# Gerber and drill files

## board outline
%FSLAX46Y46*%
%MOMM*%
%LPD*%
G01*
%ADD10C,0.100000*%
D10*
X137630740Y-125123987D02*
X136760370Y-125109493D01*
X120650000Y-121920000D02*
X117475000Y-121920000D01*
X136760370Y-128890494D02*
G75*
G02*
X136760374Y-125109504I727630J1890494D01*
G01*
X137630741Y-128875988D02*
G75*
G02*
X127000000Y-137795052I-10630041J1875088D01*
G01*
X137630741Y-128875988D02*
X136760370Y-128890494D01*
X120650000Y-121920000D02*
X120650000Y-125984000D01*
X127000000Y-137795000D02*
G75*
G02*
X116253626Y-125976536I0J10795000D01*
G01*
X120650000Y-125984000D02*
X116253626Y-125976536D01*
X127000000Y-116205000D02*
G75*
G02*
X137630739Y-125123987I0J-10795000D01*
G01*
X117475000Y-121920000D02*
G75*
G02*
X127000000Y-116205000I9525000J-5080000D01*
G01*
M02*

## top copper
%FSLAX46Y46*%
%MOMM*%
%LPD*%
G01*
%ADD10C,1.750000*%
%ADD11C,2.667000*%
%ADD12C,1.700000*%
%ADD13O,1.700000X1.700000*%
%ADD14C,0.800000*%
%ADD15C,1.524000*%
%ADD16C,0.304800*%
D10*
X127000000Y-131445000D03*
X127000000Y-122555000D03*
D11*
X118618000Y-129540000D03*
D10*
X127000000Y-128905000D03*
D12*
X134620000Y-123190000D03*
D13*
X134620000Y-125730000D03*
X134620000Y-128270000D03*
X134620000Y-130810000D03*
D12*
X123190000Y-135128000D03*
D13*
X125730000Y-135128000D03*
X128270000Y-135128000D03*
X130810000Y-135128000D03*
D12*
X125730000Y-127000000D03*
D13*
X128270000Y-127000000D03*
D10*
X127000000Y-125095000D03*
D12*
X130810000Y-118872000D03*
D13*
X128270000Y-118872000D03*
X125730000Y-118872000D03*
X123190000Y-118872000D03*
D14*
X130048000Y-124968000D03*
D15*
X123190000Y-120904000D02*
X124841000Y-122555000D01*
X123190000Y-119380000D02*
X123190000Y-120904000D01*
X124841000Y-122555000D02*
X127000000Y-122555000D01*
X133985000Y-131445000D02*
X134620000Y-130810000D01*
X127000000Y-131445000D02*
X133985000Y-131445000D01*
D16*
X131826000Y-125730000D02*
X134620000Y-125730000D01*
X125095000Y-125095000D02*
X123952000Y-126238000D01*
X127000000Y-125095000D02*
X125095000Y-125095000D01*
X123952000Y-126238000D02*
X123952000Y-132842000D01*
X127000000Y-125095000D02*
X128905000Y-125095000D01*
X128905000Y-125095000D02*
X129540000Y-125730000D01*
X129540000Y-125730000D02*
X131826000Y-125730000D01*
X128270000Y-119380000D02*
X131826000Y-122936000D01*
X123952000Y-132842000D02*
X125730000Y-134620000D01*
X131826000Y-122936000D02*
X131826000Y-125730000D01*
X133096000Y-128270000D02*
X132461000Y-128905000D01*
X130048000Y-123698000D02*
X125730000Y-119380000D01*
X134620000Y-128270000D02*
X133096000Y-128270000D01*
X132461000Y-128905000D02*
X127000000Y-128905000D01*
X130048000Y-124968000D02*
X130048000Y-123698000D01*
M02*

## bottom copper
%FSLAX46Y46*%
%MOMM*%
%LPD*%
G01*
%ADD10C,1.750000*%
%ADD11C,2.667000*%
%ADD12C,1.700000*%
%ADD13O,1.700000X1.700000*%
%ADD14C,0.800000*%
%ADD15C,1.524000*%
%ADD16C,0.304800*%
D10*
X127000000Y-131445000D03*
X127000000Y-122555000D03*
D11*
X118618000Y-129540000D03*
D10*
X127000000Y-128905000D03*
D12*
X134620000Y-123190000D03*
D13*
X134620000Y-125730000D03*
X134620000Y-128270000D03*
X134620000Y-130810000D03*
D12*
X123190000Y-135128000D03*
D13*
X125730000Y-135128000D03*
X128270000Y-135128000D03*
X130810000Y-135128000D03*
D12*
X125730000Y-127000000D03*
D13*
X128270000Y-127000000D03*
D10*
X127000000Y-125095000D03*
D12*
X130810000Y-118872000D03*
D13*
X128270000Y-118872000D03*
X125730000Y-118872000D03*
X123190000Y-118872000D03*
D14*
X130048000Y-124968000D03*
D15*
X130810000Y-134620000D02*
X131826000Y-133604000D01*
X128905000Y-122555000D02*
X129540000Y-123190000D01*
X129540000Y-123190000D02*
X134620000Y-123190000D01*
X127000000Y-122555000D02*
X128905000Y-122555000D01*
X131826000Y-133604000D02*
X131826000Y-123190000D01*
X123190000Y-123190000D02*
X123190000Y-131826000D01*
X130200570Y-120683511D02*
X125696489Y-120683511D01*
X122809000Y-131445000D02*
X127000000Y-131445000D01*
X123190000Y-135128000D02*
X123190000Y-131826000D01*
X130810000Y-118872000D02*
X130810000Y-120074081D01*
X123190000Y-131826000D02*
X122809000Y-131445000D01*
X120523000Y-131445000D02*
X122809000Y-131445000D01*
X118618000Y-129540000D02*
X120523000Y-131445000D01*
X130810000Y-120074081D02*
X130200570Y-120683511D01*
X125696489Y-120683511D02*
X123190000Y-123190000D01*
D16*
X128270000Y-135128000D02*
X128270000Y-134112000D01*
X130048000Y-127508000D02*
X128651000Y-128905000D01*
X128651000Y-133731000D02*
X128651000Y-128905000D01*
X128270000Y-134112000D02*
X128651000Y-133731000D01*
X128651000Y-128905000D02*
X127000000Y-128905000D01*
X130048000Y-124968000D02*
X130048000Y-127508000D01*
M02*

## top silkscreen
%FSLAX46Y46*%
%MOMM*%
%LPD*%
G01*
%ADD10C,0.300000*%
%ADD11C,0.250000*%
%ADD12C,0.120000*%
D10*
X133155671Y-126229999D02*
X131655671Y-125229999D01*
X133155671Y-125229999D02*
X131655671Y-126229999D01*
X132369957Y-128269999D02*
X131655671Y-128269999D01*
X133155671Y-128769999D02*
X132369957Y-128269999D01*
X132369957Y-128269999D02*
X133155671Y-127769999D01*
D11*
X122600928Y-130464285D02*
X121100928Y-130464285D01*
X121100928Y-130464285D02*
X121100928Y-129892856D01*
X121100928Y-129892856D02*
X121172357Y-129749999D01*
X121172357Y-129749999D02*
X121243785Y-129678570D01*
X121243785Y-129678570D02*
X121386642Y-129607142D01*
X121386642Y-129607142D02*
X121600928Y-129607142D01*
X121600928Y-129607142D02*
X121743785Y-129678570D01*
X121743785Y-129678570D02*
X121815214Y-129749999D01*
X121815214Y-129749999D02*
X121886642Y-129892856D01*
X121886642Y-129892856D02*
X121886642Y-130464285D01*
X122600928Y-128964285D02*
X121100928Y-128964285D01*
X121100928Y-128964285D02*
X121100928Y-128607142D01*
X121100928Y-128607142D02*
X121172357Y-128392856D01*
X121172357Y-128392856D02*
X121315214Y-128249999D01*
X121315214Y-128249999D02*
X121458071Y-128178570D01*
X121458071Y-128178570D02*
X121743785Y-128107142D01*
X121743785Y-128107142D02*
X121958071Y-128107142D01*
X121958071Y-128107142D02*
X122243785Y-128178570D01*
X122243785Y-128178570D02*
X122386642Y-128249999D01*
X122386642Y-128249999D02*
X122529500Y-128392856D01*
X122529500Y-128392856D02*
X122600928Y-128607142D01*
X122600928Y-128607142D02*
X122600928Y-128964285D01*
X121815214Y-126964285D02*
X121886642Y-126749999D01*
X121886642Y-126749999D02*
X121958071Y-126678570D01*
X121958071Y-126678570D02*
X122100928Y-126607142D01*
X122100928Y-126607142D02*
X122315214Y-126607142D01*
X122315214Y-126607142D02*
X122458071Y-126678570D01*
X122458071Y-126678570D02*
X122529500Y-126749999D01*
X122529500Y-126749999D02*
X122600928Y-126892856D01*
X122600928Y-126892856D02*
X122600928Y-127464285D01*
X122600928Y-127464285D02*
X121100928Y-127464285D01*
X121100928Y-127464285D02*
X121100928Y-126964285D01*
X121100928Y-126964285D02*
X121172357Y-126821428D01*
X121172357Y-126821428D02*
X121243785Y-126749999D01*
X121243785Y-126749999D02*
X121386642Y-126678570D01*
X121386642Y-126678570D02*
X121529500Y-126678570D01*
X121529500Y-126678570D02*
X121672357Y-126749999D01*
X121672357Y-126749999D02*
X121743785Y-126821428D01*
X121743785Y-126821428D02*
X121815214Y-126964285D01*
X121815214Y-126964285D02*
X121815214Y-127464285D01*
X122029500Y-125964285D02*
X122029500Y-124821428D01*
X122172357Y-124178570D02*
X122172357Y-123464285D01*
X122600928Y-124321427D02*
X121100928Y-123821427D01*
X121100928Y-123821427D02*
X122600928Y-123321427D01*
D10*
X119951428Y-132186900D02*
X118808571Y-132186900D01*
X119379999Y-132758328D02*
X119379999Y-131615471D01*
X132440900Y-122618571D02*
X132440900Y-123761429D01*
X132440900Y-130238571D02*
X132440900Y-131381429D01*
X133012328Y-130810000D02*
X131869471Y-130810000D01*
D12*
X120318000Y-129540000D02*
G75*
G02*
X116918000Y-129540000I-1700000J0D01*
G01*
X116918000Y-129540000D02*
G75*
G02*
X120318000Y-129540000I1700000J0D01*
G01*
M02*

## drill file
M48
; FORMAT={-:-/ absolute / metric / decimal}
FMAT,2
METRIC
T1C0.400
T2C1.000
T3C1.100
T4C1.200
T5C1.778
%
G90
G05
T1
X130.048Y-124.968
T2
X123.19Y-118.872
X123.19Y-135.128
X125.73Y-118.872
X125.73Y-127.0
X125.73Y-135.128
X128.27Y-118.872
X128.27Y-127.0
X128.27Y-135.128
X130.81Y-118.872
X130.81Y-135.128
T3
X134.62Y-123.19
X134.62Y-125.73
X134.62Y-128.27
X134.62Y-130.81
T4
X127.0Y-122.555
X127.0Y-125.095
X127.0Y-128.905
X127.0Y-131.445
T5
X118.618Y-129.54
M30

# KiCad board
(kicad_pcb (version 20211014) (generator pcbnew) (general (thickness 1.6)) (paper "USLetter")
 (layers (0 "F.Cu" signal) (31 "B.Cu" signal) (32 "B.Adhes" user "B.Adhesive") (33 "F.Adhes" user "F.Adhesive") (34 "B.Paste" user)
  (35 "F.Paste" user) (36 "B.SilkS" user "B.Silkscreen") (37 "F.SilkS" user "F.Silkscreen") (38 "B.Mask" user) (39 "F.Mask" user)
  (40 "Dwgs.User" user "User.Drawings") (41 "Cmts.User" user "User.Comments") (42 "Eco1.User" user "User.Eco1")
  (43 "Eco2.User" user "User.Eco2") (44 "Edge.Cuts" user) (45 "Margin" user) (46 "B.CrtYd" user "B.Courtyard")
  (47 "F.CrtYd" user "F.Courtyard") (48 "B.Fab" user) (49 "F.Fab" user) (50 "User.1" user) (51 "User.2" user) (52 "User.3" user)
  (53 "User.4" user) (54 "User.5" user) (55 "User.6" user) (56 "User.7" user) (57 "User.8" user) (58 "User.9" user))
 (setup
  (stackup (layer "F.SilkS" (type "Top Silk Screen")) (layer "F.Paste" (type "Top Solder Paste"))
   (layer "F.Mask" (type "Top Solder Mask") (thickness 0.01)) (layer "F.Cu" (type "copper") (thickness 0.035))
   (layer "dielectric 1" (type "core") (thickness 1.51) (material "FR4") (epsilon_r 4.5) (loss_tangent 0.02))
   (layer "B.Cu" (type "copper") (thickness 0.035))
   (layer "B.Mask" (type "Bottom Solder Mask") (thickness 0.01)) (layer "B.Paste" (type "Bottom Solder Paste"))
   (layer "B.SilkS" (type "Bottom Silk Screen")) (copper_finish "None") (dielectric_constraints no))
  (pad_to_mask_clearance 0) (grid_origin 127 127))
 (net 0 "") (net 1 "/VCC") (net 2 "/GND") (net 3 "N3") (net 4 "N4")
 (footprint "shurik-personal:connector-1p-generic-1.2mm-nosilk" (layer "F.Cu") (at 127 131.445)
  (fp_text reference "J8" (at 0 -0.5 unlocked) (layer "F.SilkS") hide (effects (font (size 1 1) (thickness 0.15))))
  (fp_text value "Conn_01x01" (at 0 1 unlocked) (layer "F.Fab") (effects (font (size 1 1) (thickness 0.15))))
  (pad "1" thru_hole circle (at 0 0) (size 1.75 1.75) (drill 1.2) (layers *.Cu *.Mask) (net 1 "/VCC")))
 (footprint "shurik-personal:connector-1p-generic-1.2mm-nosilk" (layer "F.Cu") (at 127 122.555)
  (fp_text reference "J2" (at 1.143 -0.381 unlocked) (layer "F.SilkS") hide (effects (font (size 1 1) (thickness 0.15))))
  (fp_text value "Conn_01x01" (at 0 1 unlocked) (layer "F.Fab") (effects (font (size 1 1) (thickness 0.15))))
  (pad "1" thru_hole circle (at 0 0) (size 1.75 1.75) (drill 1.2) (layers *.Cu *.Mask) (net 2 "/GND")))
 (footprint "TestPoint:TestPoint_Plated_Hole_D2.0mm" (layer "F.Cu") (at 118.618 129.54)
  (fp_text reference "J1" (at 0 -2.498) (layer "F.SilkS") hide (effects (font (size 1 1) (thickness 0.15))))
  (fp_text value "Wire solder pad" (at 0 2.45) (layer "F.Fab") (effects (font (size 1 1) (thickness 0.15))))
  (fp_circle (center 0 0) (end 0 -1.7) (layer "F.SilkS") (width 0.12) (fill none))
  (pad "1" thru_hole circle (at 0 0) (size 2.667 2.667) (drill 1.778) (layers *.Cu *.Mask) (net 1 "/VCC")))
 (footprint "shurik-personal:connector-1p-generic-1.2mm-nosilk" (layer "F.Cu") (at 127 128.905)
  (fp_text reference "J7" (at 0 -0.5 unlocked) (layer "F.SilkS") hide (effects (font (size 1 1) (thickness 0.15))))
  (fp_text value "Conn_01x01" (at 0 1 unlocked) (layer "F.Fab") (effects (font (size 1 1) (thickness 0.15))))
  (pad "1" thru_hole circle (at 0 0) (size 1.75 1.75) (drill 1.2) (layers *.Cu *.Mask) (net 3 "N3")))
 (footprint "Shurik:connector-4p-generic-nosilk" (layer "F.Cu") (at 134.62 123.19)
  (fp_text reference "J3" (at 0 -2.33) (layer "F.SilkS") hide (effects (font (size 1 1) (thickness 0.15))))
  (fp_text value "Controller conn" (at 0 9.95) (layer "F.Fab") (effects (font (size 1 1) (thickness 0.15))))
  (pad "1" thru_hole circle (at 0 0) (size 1.7 1.7) (drill 1.1) (layers *.Cu *.Mask) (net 2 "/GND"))
  (pad "2" thru_hole oval (at 0 2.54) (size 1.7 1.7) (drill 1.1) (layers *.Cu *.Mask) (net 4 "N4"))
  (pad "3" thru_hole oval (at 0 5.08) (size 1.7 1.7) (drill 1.1) (layers *.Cu *.Mask) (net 3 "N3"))
  (pad "4" thru_hole oval (at 0 7.62) (size 1.7 1.7) (drill 1.1) (layers *.Cu *.Mask) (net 1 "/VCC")))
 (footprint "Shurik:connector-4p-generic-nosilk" (layer "F.Cu") (at 123.19 135.128 90)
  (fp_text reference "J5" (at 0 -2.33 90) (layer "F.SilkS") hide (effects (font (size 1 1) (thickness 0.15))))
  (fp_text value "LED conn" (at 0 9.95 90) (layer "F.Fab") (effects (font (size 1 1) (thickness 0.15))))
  (pad "1" thru_hole circle (at 0 0 90) (size 1.7 1.7) (drill 1) (layers *.Cu *.Mask) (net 1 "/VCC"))
  (pad "2" thru_hole oval (at 0 2.54 90) (size 1.7 1.7) (drill 1) (layers *.Cu *.Mask) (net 4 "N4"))
  (pad "3" thru_hole oval (at 0 5.08 90) (size 1.7 1.7) (drill 1) (layers *.Cu *.Mask) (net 3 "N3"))
  (pad "4" thru_hole oval (at 0 7.62 90) (size 1.7 1.7) (drill 1) (layers *.Cu *.Mask) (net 2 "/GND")))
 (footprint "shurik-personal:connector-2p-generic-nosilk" (layer "F.Cu") (at 125.73 127 90)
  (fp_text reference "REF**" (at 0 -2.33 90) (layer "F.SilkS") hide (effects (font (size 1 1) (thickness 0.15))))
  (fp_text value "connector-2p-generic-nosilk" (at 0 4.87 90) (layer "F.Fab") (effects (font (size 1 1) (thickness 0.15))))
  (pad "1" thru_hole circle (at 0 0 90) (size 1.7 1.7) (drill 1) (layers *.Cu *.Mask))
  (pad "2" thru_hole oval (at 0 2.54 90) (size 1.7 1.7) (drill 1) (layers *.Cu *.Mask)))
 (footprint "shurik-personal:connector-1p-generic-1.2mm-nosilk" (layer "F.Cu") (at 127 125.095)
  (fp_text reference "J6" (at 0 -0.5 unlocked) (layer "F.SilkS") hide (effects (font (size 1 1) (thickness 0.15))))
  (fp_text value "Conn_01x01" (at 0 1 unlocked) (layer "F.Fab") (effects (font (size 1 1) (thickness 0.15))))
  (pad "1" thru_hole circle (at 0 0) (size 1.75 1.75) (drill 1.2) (layers *.Cu *.Mask) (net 4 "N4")))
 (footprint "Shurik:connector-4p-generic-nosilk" (layer "F.Cu") (at 130.81 118.872 -90)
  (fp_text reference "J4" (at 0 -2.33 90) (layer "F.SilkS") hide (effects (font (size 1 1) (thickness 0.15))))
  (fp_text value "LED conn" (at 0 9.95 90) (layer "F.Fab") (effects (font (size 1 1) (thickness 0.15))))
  (pad "1" thru_hole circle (at 0 0 270) (size 1.7 1.7) (drill 1) (layers *.Cu *.Mask) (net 1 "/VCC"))
  (pad "2" thru_hole oval (at 0 2.54 270) (size 1.7 1.7) (drill 1) (layers *.Cu *.Mask) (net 4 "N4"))
  (pad "3" thru_hole oval (at 0 5.08 270) (size 1.7 1.7) (drill 1) (layers *.Cu *.Mask) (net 3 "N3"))
  (pad "4" thru_hole oval (at 0 7.62 270) (size 1.7 1.7) (drill 1) (layers *.Cu *.Mask) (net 2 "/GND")))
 (gr_line (start 137.63074 125.123987) (end 136.76037 125.109493) (layer "Edge.Cuts") (width 0.1))
 (gr_line (start 120.65 121.92) (end 117.475 121.92) (layer "Edge.Cuts") (width 0.1))
 (gr_arc (start 136.76037 128.890494) (mid 135.462276 126.999993) (end 136.76037 125.109493) (layer "Edge.Cuts") (width 0.1))
 (gr_arc (start 137.630741 128.875988) (mid 133.938498 135.27013) (end 127 137.795) (layer "Edge.Cuts") (width 0.1))
 (gr_line (start 137.630741 128.875988) (end 136.76037 128.890494) (layer "Edge.Cuts") (width 0.1))
 (gr_line (start 120.65 121.92) (end 120.65 125.984) (layer "Edge.Cuts") (width 0.1))
 (gr_arc (start 127 137.795) (mid 119.013129 134.262356) (end 116.253626 125.976536) (layer "Edge.Cuts") (width 0.1))
 (gr_line (start 120.65 125.984) (end 116.253626 125.976536) (layer "Edge.Cuts") (width 0.1))
 (gr_arc (start 127 116.205) (mid 133.93832 118.730063) (end 137.63074 125.123987) (layer "Edge.Cuts") (width 0.1))
 (gr_arc (start 117.475 121.92) (mid 121.446017 117.743361) (end 127 116.205) (layer "Edge.Cuts") (width 0.1))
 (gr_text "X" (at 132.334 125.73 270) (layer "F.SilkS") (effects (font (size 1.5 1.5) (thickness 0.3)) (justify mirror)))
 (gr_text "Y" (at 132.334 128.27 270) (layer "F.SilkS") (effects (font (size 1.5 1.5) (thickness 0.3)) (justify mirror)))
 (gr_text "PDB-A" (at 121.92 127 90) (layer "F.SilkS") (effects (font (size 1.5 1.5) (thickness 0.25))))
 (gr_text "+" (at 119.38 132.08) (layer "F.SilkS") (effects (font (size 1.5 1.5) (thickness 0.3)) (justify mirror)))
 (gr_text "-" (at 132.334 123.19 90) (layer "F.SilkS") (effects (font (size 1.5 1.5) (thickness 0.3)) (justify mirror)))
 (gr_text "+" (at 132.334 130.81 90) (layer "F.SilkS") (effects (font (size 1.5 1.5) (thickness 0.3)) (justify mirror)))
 (segment (start 123.19 120.904) (end 124.841 122.555) (width 1.524) (layer "F.Cu") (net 2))
 (segment (start 123.19 119.38) (end 123.19 120.904) (width 1.524) (layer "F.Cu") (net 2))
 (segment (start 124.841 122.555) (end 127 122.555) (width 1.524) (layer "F.Cu") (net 2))
 (segment (start 130.81 134.62) (end 131.826 133.604) (width 1.524) (layer "B.Cu") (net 2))
 (segment (start 128.905 122.555) (end 129.54 123.19) (width 1.524) (layer "B.Cu") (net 2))
 (segment (start 129.54 123.19) (end 134.62 123.19) (width 1.524) (layer "B.Cu") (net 2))
 (segment (start 127 122.555) (end 128.905 122.555) (width 1.524) (layer "B.Cu") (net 2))
 (segment (start 131.826 133.604) (end 131.826 123.19) (width 1.524) (layer "B.Cu") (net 2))
 (segment (start 133.985 131.445) (end 134.62 130.81) (width 1.524) (layer "F.Cu") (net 1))
 (segment (start 127 131.445) (end 133.985 131.445) (width 1.524) (layer "F.Cu") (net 1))
 (segment (start 123.19 123.19) (end 123.19 131.826) (width 1.524) (layer "B.Cu") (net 1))
 (segment (start 130.20057 120.683511) (end 125.696489 120.683511) (width 1.524) (layer "B.Cu") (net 1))
 (segment (start 122.809 131.445) (end 127 131.445) (width 1.524) (layer "B.Cu") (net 1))
 (segment (start 123.19 135.128) (end 123.19 131.826) (width 1.524) (layer "B.Cu") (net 1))
 (segment (start 130.81 118.872) (end 130.81 120.074081) (width 1.524) (layer "B.Cu") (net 1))
 (segment (start 123.19 131.826) (end 122.809 131.445) (width 1.524) (layer "B.Cu") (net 1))
 (segment (start 120.523 131.445) (end 122.809 131.445) (width 1.524) (layer "B.Cu") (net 1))
 (segment (start 118.618 129.54) (end 120.523 131.445) (width 1.524) (layer "B.Cu") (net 1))
 (segment (start 130.81 120.074081) (end 130.20057 120.683511) (width 1.524) (layer "B.Cu") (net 1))
 (segment (start 125.696489 120.683511) (end 123.19 123.19) (width 1.524) (layer "B.Cu") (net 1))
 (segment (start 131.826 125.73) (end 134.62 125.73) (width 0.3048) (layer "F.Cu") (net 4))
 (segment (start 125.095 125.095) (end 123.952 126.238) (width 0.3048) (layer "F.Cu") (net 4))
 (segment (start 127 125.095) (end 125.095 125.095) (width 0.3048) (layer "F.Cu") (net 4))
 (segment (start 123.952 126.238) (end 123.952 132.842) (width 0.3048) (layer "F.Cu") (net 4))
 (segment (start 127 125.095) (end 128.905 125.095) (width 0.3048) (layer "F.Cu") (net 4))
 (segment (start 128.905 125.095) (end 129.54 125.73) (width 0.3048) (layer "F.Cu") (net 4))
 (segment (start 129.54 125.73) (end 131.826 125.73) (width 0.3048) (layer "F.Cu") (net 4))
 (segment (start 128.27 119.38) (end 131.826 122.936) (width 0.3048) (layer "F.Cu") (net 4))
 (segment (start 123.952 132.842) (end 125.73 134.62) (width 0.3048) (layer "F.Cu") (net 4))
 (segment (start 131.826 122.936) (end 131.826 125.73) (width 0.3048) (layer "F.Cu") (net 4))
 (segment (start 133.096 128.27) (end 132.461 128.905) (width 0.3048) (layer "F.Cu") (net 3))
 (segment (start 130.048 123.698) (end 125.73 119.38) (width 0.3048) (layer "F.Cu") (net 3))
 (segment (start 134.62 128.27) (end 133.096 128.27) (width 0.3048) (layer "F.Cu") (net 3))
 (segment (start 132.461 128.905) (end 127 128.905) (width 0.3048) (layer "F.Cu") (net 3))
 (segment (start 130.048 124.968) (end 130.048 123.698) (width 0.3048) (layer "F.Cu") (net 3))
 (via (at 130.048 124.968) (size 0.8) (drill 0.4) (layers "F.Cu" "B.Cu") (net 3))
 (segment (start 128.27 135.128) (end 128.27 134.112) (width 0.3048) (layer "B.Cu") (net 3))
 (segment (start 130.048 127.508) (end 128.651 128.905) (width 0.3048) (layer "B.Cu") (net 3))
 (segment (start 128.651 133.731) (end 128.651 128.905) (width 0.3048) (layer "B.Cu") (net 3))
 (segment (start 128.27 134.112) (end 128.651 133.731) (width 0.3048) (layer "B.Cu") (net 3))
 (segment (start 128.651 128.905) (end 127 128.905) (width 0.3048) (layer "B.Cu") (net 3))
 (segment (start 130.048 124.968) (end 130.048 127.508) (width 0.3048) (layer "B.Cu") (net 3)))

